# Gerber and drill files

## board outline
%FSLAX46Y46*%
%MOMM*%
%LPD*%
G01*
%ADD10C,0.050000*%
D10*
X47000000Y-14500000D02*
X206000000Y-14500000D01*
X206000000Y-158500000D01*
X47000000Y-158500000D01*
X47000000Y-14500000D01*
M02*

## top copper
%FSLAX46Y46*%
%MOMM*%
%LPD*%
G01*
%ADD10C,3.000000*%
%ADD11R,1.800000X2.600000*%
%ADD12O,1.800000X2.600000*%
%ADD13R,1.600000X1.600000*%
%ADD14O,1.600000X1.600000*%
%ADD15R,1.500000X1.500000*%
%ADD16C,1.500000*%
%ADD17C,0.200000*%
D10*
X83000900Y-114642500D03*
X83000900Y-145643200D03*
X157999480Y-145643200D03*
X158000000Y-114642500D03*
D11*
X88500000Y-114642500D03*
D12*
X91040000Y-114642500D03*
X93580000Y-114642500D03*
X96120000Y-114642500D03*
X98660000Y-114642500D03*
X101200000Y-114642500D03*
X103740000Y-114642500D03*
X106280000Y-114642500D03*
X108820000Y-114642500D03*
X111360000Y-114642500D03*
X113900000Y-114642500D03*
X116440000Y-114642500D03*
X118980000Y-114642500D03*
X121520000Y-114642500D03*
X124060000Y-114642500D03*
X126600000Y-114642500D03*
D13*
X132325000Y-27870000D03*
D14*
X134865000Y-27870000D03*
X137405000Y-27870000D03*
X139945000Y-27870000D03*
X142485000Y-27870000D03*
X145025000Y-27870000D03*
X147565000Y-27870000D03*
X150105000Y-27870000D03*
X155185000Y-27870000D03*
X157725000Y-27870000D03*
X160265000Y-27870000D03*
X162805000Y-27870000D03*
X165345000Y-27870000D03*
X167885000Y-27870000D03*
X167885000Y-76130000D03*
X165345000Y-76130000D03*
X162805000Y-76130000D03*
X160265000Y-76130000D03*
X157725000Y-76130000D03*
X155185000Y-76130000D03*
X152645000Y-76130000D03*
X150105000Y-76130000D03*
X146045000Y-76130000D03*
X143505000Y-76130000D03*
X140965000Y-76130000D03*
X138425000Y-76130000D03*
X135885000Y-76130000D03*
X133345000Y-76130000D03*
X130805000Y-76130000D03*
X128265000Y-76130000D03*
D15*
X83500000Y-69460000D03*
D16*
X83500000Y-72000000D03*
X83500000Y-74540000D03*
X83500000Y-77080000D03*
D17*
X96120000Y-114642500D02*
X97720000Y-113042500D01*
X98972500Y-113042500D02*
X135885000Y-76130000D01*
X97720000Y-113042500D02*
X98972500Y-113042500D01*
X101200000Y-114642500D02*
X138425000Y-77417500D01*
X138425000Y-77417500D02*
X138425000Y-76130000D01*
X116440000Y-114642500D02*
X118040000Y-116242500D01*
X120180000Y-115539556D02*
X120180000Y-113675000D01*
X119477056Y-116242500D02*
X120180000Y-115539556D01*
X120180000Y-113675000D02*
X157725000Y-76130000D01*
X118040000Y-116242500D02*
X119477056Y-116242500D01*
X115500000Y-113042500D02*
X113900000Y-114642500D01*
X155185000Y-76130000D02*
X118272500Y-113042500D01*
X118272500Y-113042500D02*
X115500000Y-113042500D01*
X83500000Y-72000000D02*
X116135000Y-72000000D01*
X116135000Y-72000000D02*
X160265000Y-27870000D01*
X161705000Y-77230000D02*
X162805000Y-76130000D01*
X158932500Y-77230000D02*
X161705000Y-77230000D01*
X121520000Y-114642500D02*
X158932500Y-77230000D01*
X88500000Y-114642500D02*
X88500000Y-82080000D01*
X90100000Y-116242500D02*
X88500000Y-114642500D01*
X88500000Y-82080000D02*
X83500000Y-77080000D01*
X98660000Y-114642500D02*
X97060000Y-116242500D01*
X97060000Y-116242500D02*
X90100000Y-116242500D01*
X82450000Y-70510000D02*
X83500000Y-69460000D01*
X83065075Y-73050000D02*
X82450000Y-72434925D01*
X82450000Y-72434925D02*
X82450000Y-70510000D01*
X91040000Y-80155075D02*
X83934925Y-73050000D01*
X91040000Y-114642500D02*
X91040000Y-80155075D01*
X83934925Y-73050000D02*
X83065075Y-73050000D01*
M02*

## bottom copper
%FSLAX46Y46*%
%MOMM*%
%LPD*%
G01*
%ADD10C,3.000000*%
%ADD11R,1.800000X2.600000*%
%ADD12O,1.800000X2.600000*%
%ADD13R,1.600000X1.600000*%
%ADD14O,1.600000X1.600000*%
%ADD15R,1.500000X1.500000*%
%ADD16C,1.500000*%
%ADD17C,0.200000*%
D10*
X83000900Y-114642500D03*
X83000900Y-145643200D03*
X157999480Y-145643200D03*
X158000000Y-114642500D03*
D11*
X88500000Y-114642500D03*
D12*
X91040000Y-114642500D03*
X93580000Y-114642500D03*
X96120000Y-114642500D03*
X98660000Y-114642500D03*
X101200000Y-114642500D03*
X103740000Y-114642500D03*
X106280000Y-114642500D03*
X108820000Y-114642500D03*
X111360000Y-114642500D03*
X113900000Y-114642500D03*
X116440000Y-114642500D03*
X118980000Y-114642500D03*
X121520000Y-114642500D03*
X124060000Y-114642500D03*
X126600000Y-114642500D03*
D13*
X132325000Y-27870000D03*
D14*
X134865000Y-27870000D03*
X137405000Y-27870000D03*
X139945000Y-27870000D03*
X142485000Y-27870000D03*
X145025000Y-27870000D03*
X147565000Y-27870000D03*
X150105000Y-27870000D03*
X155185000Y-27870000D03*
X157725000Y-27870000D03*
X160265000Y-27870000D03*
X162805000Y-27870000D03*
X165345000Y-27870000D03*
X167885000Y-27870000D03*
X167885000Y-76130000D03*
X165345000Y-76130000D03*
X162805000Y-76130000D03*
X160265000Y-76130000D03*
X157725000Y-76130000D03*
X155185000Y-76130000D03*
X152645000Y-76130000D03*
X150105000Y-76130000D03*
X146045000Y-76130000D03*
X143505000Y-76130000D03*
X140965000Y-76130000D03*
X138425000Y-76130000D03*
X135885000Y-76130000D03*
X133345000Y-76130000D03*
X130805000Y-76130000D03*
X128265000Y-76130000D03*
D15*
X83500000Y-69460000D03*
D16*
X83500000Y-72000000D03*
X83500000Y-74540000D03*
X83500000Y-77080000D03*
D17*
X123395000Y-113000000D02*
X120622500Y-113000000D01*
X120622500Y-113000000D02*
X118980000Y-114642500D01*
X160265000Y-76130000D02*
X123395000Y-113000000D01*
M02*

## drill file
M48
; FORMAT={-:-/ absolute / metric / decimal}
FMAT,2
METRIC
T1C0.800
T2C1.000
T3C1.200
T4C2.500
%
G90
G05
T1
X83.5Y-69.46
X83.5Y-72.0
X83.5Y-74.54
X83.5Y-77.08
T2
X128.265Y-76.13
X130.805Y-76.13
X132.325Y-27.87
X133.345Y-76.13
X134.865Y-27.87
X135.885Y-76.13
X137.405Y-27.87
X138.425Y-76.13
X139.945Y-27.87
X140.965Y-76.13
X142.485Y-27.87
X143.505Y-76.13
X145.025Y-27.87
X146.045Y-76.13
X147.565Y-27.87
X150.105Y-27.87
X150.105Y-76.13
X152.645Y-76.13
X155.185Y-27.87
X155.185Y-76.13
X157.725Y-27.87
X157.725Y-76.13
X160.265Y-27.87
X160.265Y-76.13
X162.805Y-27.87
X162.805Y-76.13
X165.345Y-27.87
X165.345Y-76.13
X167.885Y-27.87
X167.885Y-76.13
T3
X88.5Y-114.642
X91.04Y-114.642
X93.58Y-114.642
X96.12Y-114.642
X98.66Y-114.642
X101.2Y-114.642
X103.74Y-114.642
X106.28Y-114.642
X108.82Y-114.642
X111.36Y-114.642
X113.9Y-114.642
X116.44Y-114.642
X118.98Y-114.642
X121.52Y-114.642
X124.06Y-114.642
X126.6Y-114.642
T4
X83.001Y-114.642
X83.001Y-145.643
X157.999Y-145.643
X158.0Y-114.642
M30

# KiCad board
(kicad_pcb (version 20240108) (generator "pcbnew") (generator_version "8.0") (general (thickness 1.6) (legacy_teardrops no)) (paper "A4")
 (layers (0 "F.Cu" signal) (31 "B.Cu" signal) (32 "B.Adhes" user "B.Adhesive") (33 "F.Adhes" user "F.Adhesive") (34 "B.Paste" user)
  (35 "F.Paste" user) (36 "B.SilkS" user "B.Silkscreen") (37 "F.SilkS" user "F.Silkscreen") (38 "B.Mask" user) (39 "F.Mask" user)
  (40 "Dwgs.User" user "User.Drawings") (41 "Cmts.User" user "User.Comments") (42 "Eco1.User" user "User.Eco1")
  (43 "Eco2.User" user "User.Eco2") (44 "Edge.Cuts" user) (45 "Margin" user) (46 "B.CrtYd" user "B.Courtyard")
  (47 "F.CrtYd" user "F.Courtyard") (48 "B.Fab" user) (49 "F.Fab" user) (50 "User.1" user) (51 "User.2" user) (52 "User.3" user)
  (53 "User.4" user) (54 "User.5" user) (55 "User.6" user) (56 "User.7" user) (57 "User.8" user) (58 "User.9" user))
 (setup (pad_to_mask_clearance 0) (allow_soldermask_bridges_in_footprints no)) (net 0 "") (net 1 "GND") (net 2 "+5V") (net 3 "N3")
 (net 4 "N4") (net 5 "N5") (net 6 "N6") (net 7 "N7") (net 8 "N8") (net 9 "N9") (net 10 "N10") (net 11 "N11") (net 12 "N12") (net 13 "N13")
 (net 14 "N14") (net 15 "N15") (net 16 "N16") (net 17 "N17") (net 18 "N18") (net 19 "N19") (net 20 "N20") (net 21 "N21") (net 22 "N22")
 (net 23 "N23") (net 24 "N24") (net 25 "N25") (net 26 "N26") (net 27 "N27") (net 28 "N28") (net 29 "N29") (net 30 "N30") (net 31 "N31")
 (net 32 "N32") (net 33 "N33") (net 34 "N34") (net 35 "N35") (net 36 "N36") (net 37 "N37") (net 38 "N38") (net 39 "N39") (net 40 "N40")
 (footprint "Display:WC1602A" (layer "F.Cu") (at 88.5 114.6425)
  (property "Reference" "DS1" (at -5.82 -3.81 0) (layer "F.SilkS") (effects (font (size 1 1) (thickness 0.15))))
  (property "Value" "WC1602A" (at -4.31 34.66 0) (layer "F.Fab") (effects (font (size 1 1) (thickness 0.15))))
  (pad "" thru_hole circle (at -5.4991 0) (size 3 3) (drill 2.5) (layers "*.Cu" "*.Mask") (remove_unused_layers no))
  (pad "" thru_hole circle (at -5.4991 31.0007) (size 3 3) (drill 2.5) (layers "*.Cu" "*.Mask") (remove_unused_layers no))
  (pad "" thru_hole circle (at 69.49948 31.0007) (size 3 3) (drill 2.5) (layers "*.Cu" "*.Mask") (remove_unused_layers no))
  (pad "" thru_hole circle (at 69.5 0) (size 3 3) (drill 2.5) (layers "*.Cu" "*.Mask") (remove_unused_layers no))
  (pad "1" thru_hole rect (at 0 0) (size 1.8 2.6) (drill 1.2) (layers "*.Cu" "*.Mask") (remove_unused_layers no) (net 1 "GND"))
  (pad "2" thru_hole oval (at 2.54 0) (size 1.8 2.6) (drill 1.2) (layers "*.Cu" "*.Mask") (remove_unused_layers no) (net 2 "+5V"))
  (pad "3" thru_hole oval (at 5.08 0) (size 1.8 2.6) (drill 1.2) (layers "*.Cu" "*.Mask") (remove_unused_layers no) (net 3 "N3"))
  (pad "4" thru_hole oval (at 7.62 0) (size 1.8 2.6) (drill 1.2) (layers "*.Cu" "*.Mask") (remove_unused_layers no) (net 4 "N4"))
  (pad "5" thru_hole oval (at 10.16 0) (size 1.8 2.6) (drill 1.2) (layers "*.Cu" "*.Mask") (remove_unused_layers no) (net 1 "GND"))
  (pad "6" thru_hole oval (at 12.7 0) (size 1.8 2.6) (drill 1.2) (layers "*.Cu" "*.Mask") (remove_unused_layers no) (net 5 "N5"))
  (pad "7" thru_hole oval (at 15.24 0) (size 1.8 2.6) (drill 1.2) (layers "*.Cu" "*.Mask") (remove_unused_layers no) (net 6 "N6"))
  (pad "8" thru_hole oval (at 17.78 0) (size 1.8 2.6) (drill 1.2) (layers "*.Cu" "*.Mask") (remove_unused_layers no) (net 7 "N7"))
  (pad "9" thru_hole oval (at 20.32 0) (size 1.8 2.6) (drill 1.2) (layers "*.Cu" "*.Mask") (remove_unused_layers no) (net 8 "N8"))
  (pad "10" thru_hole oval (at 22.86 0) (size 1.8 2.6) (drill 1.2) (layers "*.Cu" "*.Mask") (remove_unused_layers no) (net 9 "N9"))
  (pad "11" thru_hole oval (at 25.4 0) (size 1.8 2.6) (drill 1.2) (layers "*.Cu" "*.Mask") (remove_unused_layers no) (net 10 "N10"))
  (pad "12" thru_hole oval (at 27.94 0) (size 1.8 2.6) (drill 1.2) (layers "*.Cu" "*.Mask") (remove_unused_layers no) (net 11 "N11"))
  (pad "13" thru_hole oval (at 30.48 0) (size 1.8 2.6) (drill 1.2) (layers "*.Cu" "*.Mask") (remove_unused_layers no) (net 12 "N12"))
  (pad "14" thru_hole oval (at 33.02 0) (size 1.8 2.6) (drill 1.2) (layers "*.Cu" "*.Mask") (remove_unused_layers no) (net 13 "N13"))
  (pad "15" thru_hole oval (at 35.56 0) (size 1.8 2.6) (drill 1.2) (layers "*.Cu" "*.Mask") (remove_unused_layers no) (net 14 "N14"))
  (pad "16" thru_hole oval (at 38.1 0) (size 1.8 2.6) (drill 1.2) (layers "*.Cu" "*.Mask") (remove_unused_layers no) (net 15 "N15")))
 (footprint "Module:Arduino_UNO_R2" (layer "F.Cu") (at 132.325 27.87)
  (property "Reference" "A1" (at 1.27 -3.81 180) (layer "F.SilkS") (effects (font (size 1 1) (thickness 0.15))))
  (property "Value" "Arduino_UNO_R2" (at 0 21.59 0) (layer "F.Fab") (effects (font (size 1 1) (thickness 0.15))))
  (pad "1" thru_hole rect (at 0 0 90) (size 1.6 1.6) (drill 1) (layers "*.Cu" "*.Mask") (remove_unused_layers no) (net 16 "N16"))
  (pad "2" thru_hole oval (at 2.54 0 90) (size 1.6 1.6) (drill 1) (layers "*.Cu" "*.Mask") (remove_unused_layers no) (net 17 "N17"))
  (pad "3" thru_hole oval (at 5.08 0 90) (size 1.6 1.6) (drill 1) (layers "*.Cu" "*.Mask") (remove_unused_layers no) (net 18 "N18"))
  (pad "4" thru_hole oval (at 7.62 0 90) (size 1.6 1.6) (drill 1) (layers "*.Cu" "*.Mask") (remove_unused_layers no) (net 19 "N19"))
  (pad "5" thru_hole oval (at 10.16 0 90) (size 1.6 1.6) (drill 1) (layers "*.Cu" "*.Mask") (remove_unused_layers no) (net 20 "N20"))
  (pad "6" thru_hole oval (at 12.7 0 90) (size 1.6 1.6) (drill 1) (layers "*.Cu" "*.Mask") (remove_unused_layers no) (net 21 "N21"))
  (pad "7" thru_hole oval (at 15.24 0 90) (size 1.6 1.6) (drill 1) (layers "*.Cu" "*.Mask") (remove_unused_layers no) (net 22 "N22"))
  (pad "8" thru_hole oval (at 17.78 0 90) (size 1.6 1.6) (drill 1) (layers "*.Cu" "*.Mask") (remove_unused_layers no) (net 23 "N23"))
  (pad "9" thru_hole oval (at 22.86 0 90) (size 1.6 1.6) (drill 1) (layers "*.Cu" "*.Mask") (remove_unused_layers no) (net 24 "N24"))
  (pad "10" thru_hole oval (at 25.4 0 90) (size 1.6 1.6) (drill 1) (layers "*.Cu" "*.Mask") (remove_unused_layers no) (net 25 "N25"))
  (pad "11" thru_hole oval (at 27.94 0 90) (size 1.6 1.6) (drill 1) (layers "*.Cu" "*.Mask") (remove_unused_layers no) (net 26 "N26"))
  (pad "12" thru_hole oval (at 30.48 0 90) (size 1.6 1.6) (drill 1) (layers "*.Cu" "*.Mask") (remove_unused_layers no) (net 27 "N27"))
  (pad "13" thru_hole oval (at 33.02 0 90) (size 1.6 1.6) (drill 1) (layers "*.Cu" "*.Mask") (remove_unused_layers no) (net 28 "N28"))
  (pad "14" thru_hole oval (at 35.56 0 90) (size 1.6 1.6) (drill 1) (layers "*.Cu" "*.Mask") (remove_unused_layers no) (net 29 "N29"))
  (pad "15" thru_hole oval (at 35.56 48.26 90) (size 1.6 1.6) (drill 1) (layers "*.Cu" "*.Mask") (remove_unused_layers no) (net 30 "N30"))
  (pad "16" thru_hole oval (at 33.02 48.26 90) (size 1.6 1.6) (drill 1) (layers "*.Cu" "*.Mask") (remove_unused_layers no) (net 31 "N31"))
  (pad "17" thru_hole oval (at 30.48 48.26 90) (size 1.6 1.6) (drill 1) (layers "*.Cu" "*.Mask") (remove_unused_layers no) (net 13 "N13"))
  (pad "18" thru_hole oval (at 27.94 48.26 90) (size 1.6 1.6) (drill 1) (layers "*.Cu" "*.Mask") (remove_unused_layers no) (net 12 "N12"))
  (pad "19" thru_hole oval (at 25.4 48.26 90) (size 1.6 1.6) (drill 1) (layers "*.Cu" "*.Mask") (remove_unused_layers no) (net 11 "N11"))
  (pad "20" thru_hole oval (at 22.86 48.26 90) (size 1.6 1.6) (drill 1) (layers "*.Cu" "*.Mask") (remove_unused_layers no) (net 10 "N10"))
  (pad "21" thru_hole oval (at 20.32 48.26 90) (size 1.6 1.6) (drill 1) (layers "*.Cu" "*.Mask") (remove_unused_layers no) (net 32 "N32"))
  (pad "22" thru_hole oval (at 17.78 48.26 90) (size 1.6 1.6) (drill 1) (layers "*.Cu" "*.Mask") (remove_unused_layers no) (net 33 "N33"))
  (pad "23" thru_hole oval (at 13.72 48.26 90) (size 1.6 1.6) (drill 1) (layers "*.Cu" "*.Mask") (remove_unused_layers no) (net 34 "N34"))
  (pad "24" thru_hole oval (at 11.18 48.26 90) (size 1.6 1.6) (drill 1) (layers "*.Cu" "*.Mask") (remove_unused_layers no) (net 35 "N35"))
  (pad "25" thru_hole oval (at 8.64 48.26 90) (size 1.6 1.6) (drill 1) (layers "*.Cu" "*.Mask") (remove_unused_layers no) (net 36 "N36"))
  (pad "26" thru_hole oval (at 6.1 48.26 90) (size 1.6 1.6) (drill 1) (layers "*.Cu" "*.Mask") (remove_unused_layers no) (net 5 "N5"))
  (pad "27" thru_hole oval (at 3.56 48.26 90) (size 1.6 1.6) (drill 1) (layers "*.Cu" "*.Mask") (remove_unused_layers no) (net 4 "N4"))
  (pad "28" thru_hole oval (at 1.02 48.26 90) (size 1.6 1.6) (drill 1) (layers "*.Cu" "*.Mask") (remove_unused_layers no) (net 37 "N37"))
  (pad "29" thru_hole oval (at -1.52 48.26 90) (size 1.6 1.6) (drill 1) (layers "*.Cu" "*.Mask") (remove_unused_layers no) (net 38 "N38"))
  (pad "30" thru_hole oval (at -4.06 48.26 90) (size 1.6 1.6) (drill 1) (layers "*.Cu" "*.Mask") (remove_unused_layers no) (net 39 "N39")))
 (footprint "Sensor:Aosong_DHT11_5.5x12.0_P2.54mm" (layer "F.Cu") (at 83.5 69.46)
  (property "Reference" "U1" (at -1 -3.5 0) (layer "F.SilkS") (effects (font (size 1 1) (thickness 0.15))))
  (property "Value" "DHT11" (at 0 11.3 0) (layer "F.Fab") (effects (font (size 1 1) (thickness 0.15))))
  (pad "1" thru_hole rect (at 0 0) (size 1.5 1.5) (drill 0.8) (layers "*.Cu" "*.Mask") (remove_unused_layers no) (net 2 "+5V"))
  (pad "2" thru_hole circle (at 0 2.54) (size 1.5 1.5) (drill 0.8) (layers "*.Cu" "*.Mask") (remove_unused_layers no) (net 26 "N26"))
  (pad "3" thru_hole circle (at 0 5.08) (size 1.5 1.5) (drill 0.8) (layers "*.Cu" "*.Mask") (remove_unused_layers no) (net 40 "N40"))
  (pad "4" thru_hole circle (at 0 7.62) (size 1.5 1.5) (drill 0.8) (layers "*.Cu" "*.Mask") (remove_unused_layers no) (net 1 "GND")))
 (gr_rect (start 47 14.5) (end 206 158.5) (stroke (width 0.05) (type default)) (fill none) (layer "Edge.Cuts"))
 (segment (start 96.12 114.6425) (end 97.72 113.0425) (width 0.2) (layer "F.Cu") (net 4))
 (segment (start 98.9725 113.0425) (end 135.885 76.13) (width 0.2) (layer "F.Cu") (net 4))
 (segment (start 97.72 113.0425) (end 98.9725 113.0425) (width 0.2) (layer "F.Cu") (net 4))
 (segment (start 101.2 114.6425) (end 138.425 77.4175) (width 0.2) (layer "F.Cu") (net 5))
 (segment (start 138.425 77.4175) (end 138.425 76.13) (width 0.2) (layer "F.Cu") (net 5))
 (segment (start 116.44 114.6425) (end 118.04 116.2425) (width 0.2) (layer "F.Cu") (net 11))
 (segment (start 120.18 115.539556) (end 120.18 113.675) (width 0.2) (layer "F.Cu") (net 11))
 (segment (start 119.477056 116.2425) (end 120.18 115.539556) (width 0.2) (layer "F.Cu") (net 11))
 (segment (start 120.18 113.675) (end 157.725 76.13) (width 0.2) (layer "F.Cu") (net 11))
 (segment (start 118.04 116.2425) (end 119.477056 116.2425) (width 0.2) (layer "F.Cu") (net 11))
 (segment (start 123.395 113) (end 120.6225 113) (width 0.2) (layer "B.Cu") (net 12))
 (segment (start 120.6225 113) (end 118.98 114.6425) (width 0.2) (layer "B.Cu") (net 12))
 (segment (start 160.265 76.13) (end 123.395 113) (width 0.2) (layer "B.Cu") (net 12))
 (segment (start 115.5 113.0425) (end 113.9 114.6425) (width 0.2) (layer "F.Cu") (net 10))
 (segment (start 155.185 76.13) (end 118.2725 113.0425) (width 0.2) (layer "F.Cu") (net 10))
 (segment (start 118.2725 113.0425) (end 115.5 113.0425) (width 0.2) (layer "F.Cu") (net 10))
 (segment (start 83.5 72) (end 116.135 72) (width 0.2) (layer "F.Cu") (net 26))
 (segment (start 116.135 72) (end 160.265 27.87) (width 0.2) (layer "F.Cu") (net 26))
 (segment (start 161.705 77.23) (end 162.805 76.13) (width 0.2) (layer "F.Cu") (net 13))
 (segment (start 158.9325 77.23) (end 161.705 77.23) (width 0.2) (layer "F.Cu") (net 13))
 (segment (start 121.52 114.6425) (end 158.9325 77.23) (width 0.2) (layer "F.Cu") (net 13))
 (segment (start 88.5 114.6425) (end 88.5 82.08) (width 0.2) (layer "F.Cu") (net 1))
 (segment (start 90.1 116.2425) (end 88.5 114.6425) (width 0.2) (layer "F.Cu") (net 1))
 (segment (start 88.5 82.08) (end 83.5 77.08) (width 0.2) (layer "F.Cu") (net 1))
 (segment (start 98.66 114.6425) (end 97.06 116.2425) (width 0.2) (layer "F.Cu") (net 1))
 (segment (start 97.06 116.2425) (end 90.1 116.2425) (width 0.2) (layer "F.Cu") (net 1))
 (segment (start 82.45 70.51) (end 83.5 69.46) (width 0.2) (layer "F.Cu") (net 2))
 (segment (start 83.065075 73.05) (end 82.45 72.434925) (width 0.2) (layer "F.Cu") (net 2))
 (segment (start 82.45 72.434925) (end 82.45 70.51) (width 0.2) (layer "F.Cu") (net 2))
 (segment (start 91.04 80.155075) (end 83.934925 73.05) (width 0.2) (layer "F.Cu") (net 2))
 (segment (start 91.04 114.6425) (end 91.04 80.155075) (width 0.2) (layer "F.Cu") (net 2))
 (segment (start 83.934925 73.05) (end 83.065075 73.05) (width 0.2) (layer "F.Cu") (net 2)))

